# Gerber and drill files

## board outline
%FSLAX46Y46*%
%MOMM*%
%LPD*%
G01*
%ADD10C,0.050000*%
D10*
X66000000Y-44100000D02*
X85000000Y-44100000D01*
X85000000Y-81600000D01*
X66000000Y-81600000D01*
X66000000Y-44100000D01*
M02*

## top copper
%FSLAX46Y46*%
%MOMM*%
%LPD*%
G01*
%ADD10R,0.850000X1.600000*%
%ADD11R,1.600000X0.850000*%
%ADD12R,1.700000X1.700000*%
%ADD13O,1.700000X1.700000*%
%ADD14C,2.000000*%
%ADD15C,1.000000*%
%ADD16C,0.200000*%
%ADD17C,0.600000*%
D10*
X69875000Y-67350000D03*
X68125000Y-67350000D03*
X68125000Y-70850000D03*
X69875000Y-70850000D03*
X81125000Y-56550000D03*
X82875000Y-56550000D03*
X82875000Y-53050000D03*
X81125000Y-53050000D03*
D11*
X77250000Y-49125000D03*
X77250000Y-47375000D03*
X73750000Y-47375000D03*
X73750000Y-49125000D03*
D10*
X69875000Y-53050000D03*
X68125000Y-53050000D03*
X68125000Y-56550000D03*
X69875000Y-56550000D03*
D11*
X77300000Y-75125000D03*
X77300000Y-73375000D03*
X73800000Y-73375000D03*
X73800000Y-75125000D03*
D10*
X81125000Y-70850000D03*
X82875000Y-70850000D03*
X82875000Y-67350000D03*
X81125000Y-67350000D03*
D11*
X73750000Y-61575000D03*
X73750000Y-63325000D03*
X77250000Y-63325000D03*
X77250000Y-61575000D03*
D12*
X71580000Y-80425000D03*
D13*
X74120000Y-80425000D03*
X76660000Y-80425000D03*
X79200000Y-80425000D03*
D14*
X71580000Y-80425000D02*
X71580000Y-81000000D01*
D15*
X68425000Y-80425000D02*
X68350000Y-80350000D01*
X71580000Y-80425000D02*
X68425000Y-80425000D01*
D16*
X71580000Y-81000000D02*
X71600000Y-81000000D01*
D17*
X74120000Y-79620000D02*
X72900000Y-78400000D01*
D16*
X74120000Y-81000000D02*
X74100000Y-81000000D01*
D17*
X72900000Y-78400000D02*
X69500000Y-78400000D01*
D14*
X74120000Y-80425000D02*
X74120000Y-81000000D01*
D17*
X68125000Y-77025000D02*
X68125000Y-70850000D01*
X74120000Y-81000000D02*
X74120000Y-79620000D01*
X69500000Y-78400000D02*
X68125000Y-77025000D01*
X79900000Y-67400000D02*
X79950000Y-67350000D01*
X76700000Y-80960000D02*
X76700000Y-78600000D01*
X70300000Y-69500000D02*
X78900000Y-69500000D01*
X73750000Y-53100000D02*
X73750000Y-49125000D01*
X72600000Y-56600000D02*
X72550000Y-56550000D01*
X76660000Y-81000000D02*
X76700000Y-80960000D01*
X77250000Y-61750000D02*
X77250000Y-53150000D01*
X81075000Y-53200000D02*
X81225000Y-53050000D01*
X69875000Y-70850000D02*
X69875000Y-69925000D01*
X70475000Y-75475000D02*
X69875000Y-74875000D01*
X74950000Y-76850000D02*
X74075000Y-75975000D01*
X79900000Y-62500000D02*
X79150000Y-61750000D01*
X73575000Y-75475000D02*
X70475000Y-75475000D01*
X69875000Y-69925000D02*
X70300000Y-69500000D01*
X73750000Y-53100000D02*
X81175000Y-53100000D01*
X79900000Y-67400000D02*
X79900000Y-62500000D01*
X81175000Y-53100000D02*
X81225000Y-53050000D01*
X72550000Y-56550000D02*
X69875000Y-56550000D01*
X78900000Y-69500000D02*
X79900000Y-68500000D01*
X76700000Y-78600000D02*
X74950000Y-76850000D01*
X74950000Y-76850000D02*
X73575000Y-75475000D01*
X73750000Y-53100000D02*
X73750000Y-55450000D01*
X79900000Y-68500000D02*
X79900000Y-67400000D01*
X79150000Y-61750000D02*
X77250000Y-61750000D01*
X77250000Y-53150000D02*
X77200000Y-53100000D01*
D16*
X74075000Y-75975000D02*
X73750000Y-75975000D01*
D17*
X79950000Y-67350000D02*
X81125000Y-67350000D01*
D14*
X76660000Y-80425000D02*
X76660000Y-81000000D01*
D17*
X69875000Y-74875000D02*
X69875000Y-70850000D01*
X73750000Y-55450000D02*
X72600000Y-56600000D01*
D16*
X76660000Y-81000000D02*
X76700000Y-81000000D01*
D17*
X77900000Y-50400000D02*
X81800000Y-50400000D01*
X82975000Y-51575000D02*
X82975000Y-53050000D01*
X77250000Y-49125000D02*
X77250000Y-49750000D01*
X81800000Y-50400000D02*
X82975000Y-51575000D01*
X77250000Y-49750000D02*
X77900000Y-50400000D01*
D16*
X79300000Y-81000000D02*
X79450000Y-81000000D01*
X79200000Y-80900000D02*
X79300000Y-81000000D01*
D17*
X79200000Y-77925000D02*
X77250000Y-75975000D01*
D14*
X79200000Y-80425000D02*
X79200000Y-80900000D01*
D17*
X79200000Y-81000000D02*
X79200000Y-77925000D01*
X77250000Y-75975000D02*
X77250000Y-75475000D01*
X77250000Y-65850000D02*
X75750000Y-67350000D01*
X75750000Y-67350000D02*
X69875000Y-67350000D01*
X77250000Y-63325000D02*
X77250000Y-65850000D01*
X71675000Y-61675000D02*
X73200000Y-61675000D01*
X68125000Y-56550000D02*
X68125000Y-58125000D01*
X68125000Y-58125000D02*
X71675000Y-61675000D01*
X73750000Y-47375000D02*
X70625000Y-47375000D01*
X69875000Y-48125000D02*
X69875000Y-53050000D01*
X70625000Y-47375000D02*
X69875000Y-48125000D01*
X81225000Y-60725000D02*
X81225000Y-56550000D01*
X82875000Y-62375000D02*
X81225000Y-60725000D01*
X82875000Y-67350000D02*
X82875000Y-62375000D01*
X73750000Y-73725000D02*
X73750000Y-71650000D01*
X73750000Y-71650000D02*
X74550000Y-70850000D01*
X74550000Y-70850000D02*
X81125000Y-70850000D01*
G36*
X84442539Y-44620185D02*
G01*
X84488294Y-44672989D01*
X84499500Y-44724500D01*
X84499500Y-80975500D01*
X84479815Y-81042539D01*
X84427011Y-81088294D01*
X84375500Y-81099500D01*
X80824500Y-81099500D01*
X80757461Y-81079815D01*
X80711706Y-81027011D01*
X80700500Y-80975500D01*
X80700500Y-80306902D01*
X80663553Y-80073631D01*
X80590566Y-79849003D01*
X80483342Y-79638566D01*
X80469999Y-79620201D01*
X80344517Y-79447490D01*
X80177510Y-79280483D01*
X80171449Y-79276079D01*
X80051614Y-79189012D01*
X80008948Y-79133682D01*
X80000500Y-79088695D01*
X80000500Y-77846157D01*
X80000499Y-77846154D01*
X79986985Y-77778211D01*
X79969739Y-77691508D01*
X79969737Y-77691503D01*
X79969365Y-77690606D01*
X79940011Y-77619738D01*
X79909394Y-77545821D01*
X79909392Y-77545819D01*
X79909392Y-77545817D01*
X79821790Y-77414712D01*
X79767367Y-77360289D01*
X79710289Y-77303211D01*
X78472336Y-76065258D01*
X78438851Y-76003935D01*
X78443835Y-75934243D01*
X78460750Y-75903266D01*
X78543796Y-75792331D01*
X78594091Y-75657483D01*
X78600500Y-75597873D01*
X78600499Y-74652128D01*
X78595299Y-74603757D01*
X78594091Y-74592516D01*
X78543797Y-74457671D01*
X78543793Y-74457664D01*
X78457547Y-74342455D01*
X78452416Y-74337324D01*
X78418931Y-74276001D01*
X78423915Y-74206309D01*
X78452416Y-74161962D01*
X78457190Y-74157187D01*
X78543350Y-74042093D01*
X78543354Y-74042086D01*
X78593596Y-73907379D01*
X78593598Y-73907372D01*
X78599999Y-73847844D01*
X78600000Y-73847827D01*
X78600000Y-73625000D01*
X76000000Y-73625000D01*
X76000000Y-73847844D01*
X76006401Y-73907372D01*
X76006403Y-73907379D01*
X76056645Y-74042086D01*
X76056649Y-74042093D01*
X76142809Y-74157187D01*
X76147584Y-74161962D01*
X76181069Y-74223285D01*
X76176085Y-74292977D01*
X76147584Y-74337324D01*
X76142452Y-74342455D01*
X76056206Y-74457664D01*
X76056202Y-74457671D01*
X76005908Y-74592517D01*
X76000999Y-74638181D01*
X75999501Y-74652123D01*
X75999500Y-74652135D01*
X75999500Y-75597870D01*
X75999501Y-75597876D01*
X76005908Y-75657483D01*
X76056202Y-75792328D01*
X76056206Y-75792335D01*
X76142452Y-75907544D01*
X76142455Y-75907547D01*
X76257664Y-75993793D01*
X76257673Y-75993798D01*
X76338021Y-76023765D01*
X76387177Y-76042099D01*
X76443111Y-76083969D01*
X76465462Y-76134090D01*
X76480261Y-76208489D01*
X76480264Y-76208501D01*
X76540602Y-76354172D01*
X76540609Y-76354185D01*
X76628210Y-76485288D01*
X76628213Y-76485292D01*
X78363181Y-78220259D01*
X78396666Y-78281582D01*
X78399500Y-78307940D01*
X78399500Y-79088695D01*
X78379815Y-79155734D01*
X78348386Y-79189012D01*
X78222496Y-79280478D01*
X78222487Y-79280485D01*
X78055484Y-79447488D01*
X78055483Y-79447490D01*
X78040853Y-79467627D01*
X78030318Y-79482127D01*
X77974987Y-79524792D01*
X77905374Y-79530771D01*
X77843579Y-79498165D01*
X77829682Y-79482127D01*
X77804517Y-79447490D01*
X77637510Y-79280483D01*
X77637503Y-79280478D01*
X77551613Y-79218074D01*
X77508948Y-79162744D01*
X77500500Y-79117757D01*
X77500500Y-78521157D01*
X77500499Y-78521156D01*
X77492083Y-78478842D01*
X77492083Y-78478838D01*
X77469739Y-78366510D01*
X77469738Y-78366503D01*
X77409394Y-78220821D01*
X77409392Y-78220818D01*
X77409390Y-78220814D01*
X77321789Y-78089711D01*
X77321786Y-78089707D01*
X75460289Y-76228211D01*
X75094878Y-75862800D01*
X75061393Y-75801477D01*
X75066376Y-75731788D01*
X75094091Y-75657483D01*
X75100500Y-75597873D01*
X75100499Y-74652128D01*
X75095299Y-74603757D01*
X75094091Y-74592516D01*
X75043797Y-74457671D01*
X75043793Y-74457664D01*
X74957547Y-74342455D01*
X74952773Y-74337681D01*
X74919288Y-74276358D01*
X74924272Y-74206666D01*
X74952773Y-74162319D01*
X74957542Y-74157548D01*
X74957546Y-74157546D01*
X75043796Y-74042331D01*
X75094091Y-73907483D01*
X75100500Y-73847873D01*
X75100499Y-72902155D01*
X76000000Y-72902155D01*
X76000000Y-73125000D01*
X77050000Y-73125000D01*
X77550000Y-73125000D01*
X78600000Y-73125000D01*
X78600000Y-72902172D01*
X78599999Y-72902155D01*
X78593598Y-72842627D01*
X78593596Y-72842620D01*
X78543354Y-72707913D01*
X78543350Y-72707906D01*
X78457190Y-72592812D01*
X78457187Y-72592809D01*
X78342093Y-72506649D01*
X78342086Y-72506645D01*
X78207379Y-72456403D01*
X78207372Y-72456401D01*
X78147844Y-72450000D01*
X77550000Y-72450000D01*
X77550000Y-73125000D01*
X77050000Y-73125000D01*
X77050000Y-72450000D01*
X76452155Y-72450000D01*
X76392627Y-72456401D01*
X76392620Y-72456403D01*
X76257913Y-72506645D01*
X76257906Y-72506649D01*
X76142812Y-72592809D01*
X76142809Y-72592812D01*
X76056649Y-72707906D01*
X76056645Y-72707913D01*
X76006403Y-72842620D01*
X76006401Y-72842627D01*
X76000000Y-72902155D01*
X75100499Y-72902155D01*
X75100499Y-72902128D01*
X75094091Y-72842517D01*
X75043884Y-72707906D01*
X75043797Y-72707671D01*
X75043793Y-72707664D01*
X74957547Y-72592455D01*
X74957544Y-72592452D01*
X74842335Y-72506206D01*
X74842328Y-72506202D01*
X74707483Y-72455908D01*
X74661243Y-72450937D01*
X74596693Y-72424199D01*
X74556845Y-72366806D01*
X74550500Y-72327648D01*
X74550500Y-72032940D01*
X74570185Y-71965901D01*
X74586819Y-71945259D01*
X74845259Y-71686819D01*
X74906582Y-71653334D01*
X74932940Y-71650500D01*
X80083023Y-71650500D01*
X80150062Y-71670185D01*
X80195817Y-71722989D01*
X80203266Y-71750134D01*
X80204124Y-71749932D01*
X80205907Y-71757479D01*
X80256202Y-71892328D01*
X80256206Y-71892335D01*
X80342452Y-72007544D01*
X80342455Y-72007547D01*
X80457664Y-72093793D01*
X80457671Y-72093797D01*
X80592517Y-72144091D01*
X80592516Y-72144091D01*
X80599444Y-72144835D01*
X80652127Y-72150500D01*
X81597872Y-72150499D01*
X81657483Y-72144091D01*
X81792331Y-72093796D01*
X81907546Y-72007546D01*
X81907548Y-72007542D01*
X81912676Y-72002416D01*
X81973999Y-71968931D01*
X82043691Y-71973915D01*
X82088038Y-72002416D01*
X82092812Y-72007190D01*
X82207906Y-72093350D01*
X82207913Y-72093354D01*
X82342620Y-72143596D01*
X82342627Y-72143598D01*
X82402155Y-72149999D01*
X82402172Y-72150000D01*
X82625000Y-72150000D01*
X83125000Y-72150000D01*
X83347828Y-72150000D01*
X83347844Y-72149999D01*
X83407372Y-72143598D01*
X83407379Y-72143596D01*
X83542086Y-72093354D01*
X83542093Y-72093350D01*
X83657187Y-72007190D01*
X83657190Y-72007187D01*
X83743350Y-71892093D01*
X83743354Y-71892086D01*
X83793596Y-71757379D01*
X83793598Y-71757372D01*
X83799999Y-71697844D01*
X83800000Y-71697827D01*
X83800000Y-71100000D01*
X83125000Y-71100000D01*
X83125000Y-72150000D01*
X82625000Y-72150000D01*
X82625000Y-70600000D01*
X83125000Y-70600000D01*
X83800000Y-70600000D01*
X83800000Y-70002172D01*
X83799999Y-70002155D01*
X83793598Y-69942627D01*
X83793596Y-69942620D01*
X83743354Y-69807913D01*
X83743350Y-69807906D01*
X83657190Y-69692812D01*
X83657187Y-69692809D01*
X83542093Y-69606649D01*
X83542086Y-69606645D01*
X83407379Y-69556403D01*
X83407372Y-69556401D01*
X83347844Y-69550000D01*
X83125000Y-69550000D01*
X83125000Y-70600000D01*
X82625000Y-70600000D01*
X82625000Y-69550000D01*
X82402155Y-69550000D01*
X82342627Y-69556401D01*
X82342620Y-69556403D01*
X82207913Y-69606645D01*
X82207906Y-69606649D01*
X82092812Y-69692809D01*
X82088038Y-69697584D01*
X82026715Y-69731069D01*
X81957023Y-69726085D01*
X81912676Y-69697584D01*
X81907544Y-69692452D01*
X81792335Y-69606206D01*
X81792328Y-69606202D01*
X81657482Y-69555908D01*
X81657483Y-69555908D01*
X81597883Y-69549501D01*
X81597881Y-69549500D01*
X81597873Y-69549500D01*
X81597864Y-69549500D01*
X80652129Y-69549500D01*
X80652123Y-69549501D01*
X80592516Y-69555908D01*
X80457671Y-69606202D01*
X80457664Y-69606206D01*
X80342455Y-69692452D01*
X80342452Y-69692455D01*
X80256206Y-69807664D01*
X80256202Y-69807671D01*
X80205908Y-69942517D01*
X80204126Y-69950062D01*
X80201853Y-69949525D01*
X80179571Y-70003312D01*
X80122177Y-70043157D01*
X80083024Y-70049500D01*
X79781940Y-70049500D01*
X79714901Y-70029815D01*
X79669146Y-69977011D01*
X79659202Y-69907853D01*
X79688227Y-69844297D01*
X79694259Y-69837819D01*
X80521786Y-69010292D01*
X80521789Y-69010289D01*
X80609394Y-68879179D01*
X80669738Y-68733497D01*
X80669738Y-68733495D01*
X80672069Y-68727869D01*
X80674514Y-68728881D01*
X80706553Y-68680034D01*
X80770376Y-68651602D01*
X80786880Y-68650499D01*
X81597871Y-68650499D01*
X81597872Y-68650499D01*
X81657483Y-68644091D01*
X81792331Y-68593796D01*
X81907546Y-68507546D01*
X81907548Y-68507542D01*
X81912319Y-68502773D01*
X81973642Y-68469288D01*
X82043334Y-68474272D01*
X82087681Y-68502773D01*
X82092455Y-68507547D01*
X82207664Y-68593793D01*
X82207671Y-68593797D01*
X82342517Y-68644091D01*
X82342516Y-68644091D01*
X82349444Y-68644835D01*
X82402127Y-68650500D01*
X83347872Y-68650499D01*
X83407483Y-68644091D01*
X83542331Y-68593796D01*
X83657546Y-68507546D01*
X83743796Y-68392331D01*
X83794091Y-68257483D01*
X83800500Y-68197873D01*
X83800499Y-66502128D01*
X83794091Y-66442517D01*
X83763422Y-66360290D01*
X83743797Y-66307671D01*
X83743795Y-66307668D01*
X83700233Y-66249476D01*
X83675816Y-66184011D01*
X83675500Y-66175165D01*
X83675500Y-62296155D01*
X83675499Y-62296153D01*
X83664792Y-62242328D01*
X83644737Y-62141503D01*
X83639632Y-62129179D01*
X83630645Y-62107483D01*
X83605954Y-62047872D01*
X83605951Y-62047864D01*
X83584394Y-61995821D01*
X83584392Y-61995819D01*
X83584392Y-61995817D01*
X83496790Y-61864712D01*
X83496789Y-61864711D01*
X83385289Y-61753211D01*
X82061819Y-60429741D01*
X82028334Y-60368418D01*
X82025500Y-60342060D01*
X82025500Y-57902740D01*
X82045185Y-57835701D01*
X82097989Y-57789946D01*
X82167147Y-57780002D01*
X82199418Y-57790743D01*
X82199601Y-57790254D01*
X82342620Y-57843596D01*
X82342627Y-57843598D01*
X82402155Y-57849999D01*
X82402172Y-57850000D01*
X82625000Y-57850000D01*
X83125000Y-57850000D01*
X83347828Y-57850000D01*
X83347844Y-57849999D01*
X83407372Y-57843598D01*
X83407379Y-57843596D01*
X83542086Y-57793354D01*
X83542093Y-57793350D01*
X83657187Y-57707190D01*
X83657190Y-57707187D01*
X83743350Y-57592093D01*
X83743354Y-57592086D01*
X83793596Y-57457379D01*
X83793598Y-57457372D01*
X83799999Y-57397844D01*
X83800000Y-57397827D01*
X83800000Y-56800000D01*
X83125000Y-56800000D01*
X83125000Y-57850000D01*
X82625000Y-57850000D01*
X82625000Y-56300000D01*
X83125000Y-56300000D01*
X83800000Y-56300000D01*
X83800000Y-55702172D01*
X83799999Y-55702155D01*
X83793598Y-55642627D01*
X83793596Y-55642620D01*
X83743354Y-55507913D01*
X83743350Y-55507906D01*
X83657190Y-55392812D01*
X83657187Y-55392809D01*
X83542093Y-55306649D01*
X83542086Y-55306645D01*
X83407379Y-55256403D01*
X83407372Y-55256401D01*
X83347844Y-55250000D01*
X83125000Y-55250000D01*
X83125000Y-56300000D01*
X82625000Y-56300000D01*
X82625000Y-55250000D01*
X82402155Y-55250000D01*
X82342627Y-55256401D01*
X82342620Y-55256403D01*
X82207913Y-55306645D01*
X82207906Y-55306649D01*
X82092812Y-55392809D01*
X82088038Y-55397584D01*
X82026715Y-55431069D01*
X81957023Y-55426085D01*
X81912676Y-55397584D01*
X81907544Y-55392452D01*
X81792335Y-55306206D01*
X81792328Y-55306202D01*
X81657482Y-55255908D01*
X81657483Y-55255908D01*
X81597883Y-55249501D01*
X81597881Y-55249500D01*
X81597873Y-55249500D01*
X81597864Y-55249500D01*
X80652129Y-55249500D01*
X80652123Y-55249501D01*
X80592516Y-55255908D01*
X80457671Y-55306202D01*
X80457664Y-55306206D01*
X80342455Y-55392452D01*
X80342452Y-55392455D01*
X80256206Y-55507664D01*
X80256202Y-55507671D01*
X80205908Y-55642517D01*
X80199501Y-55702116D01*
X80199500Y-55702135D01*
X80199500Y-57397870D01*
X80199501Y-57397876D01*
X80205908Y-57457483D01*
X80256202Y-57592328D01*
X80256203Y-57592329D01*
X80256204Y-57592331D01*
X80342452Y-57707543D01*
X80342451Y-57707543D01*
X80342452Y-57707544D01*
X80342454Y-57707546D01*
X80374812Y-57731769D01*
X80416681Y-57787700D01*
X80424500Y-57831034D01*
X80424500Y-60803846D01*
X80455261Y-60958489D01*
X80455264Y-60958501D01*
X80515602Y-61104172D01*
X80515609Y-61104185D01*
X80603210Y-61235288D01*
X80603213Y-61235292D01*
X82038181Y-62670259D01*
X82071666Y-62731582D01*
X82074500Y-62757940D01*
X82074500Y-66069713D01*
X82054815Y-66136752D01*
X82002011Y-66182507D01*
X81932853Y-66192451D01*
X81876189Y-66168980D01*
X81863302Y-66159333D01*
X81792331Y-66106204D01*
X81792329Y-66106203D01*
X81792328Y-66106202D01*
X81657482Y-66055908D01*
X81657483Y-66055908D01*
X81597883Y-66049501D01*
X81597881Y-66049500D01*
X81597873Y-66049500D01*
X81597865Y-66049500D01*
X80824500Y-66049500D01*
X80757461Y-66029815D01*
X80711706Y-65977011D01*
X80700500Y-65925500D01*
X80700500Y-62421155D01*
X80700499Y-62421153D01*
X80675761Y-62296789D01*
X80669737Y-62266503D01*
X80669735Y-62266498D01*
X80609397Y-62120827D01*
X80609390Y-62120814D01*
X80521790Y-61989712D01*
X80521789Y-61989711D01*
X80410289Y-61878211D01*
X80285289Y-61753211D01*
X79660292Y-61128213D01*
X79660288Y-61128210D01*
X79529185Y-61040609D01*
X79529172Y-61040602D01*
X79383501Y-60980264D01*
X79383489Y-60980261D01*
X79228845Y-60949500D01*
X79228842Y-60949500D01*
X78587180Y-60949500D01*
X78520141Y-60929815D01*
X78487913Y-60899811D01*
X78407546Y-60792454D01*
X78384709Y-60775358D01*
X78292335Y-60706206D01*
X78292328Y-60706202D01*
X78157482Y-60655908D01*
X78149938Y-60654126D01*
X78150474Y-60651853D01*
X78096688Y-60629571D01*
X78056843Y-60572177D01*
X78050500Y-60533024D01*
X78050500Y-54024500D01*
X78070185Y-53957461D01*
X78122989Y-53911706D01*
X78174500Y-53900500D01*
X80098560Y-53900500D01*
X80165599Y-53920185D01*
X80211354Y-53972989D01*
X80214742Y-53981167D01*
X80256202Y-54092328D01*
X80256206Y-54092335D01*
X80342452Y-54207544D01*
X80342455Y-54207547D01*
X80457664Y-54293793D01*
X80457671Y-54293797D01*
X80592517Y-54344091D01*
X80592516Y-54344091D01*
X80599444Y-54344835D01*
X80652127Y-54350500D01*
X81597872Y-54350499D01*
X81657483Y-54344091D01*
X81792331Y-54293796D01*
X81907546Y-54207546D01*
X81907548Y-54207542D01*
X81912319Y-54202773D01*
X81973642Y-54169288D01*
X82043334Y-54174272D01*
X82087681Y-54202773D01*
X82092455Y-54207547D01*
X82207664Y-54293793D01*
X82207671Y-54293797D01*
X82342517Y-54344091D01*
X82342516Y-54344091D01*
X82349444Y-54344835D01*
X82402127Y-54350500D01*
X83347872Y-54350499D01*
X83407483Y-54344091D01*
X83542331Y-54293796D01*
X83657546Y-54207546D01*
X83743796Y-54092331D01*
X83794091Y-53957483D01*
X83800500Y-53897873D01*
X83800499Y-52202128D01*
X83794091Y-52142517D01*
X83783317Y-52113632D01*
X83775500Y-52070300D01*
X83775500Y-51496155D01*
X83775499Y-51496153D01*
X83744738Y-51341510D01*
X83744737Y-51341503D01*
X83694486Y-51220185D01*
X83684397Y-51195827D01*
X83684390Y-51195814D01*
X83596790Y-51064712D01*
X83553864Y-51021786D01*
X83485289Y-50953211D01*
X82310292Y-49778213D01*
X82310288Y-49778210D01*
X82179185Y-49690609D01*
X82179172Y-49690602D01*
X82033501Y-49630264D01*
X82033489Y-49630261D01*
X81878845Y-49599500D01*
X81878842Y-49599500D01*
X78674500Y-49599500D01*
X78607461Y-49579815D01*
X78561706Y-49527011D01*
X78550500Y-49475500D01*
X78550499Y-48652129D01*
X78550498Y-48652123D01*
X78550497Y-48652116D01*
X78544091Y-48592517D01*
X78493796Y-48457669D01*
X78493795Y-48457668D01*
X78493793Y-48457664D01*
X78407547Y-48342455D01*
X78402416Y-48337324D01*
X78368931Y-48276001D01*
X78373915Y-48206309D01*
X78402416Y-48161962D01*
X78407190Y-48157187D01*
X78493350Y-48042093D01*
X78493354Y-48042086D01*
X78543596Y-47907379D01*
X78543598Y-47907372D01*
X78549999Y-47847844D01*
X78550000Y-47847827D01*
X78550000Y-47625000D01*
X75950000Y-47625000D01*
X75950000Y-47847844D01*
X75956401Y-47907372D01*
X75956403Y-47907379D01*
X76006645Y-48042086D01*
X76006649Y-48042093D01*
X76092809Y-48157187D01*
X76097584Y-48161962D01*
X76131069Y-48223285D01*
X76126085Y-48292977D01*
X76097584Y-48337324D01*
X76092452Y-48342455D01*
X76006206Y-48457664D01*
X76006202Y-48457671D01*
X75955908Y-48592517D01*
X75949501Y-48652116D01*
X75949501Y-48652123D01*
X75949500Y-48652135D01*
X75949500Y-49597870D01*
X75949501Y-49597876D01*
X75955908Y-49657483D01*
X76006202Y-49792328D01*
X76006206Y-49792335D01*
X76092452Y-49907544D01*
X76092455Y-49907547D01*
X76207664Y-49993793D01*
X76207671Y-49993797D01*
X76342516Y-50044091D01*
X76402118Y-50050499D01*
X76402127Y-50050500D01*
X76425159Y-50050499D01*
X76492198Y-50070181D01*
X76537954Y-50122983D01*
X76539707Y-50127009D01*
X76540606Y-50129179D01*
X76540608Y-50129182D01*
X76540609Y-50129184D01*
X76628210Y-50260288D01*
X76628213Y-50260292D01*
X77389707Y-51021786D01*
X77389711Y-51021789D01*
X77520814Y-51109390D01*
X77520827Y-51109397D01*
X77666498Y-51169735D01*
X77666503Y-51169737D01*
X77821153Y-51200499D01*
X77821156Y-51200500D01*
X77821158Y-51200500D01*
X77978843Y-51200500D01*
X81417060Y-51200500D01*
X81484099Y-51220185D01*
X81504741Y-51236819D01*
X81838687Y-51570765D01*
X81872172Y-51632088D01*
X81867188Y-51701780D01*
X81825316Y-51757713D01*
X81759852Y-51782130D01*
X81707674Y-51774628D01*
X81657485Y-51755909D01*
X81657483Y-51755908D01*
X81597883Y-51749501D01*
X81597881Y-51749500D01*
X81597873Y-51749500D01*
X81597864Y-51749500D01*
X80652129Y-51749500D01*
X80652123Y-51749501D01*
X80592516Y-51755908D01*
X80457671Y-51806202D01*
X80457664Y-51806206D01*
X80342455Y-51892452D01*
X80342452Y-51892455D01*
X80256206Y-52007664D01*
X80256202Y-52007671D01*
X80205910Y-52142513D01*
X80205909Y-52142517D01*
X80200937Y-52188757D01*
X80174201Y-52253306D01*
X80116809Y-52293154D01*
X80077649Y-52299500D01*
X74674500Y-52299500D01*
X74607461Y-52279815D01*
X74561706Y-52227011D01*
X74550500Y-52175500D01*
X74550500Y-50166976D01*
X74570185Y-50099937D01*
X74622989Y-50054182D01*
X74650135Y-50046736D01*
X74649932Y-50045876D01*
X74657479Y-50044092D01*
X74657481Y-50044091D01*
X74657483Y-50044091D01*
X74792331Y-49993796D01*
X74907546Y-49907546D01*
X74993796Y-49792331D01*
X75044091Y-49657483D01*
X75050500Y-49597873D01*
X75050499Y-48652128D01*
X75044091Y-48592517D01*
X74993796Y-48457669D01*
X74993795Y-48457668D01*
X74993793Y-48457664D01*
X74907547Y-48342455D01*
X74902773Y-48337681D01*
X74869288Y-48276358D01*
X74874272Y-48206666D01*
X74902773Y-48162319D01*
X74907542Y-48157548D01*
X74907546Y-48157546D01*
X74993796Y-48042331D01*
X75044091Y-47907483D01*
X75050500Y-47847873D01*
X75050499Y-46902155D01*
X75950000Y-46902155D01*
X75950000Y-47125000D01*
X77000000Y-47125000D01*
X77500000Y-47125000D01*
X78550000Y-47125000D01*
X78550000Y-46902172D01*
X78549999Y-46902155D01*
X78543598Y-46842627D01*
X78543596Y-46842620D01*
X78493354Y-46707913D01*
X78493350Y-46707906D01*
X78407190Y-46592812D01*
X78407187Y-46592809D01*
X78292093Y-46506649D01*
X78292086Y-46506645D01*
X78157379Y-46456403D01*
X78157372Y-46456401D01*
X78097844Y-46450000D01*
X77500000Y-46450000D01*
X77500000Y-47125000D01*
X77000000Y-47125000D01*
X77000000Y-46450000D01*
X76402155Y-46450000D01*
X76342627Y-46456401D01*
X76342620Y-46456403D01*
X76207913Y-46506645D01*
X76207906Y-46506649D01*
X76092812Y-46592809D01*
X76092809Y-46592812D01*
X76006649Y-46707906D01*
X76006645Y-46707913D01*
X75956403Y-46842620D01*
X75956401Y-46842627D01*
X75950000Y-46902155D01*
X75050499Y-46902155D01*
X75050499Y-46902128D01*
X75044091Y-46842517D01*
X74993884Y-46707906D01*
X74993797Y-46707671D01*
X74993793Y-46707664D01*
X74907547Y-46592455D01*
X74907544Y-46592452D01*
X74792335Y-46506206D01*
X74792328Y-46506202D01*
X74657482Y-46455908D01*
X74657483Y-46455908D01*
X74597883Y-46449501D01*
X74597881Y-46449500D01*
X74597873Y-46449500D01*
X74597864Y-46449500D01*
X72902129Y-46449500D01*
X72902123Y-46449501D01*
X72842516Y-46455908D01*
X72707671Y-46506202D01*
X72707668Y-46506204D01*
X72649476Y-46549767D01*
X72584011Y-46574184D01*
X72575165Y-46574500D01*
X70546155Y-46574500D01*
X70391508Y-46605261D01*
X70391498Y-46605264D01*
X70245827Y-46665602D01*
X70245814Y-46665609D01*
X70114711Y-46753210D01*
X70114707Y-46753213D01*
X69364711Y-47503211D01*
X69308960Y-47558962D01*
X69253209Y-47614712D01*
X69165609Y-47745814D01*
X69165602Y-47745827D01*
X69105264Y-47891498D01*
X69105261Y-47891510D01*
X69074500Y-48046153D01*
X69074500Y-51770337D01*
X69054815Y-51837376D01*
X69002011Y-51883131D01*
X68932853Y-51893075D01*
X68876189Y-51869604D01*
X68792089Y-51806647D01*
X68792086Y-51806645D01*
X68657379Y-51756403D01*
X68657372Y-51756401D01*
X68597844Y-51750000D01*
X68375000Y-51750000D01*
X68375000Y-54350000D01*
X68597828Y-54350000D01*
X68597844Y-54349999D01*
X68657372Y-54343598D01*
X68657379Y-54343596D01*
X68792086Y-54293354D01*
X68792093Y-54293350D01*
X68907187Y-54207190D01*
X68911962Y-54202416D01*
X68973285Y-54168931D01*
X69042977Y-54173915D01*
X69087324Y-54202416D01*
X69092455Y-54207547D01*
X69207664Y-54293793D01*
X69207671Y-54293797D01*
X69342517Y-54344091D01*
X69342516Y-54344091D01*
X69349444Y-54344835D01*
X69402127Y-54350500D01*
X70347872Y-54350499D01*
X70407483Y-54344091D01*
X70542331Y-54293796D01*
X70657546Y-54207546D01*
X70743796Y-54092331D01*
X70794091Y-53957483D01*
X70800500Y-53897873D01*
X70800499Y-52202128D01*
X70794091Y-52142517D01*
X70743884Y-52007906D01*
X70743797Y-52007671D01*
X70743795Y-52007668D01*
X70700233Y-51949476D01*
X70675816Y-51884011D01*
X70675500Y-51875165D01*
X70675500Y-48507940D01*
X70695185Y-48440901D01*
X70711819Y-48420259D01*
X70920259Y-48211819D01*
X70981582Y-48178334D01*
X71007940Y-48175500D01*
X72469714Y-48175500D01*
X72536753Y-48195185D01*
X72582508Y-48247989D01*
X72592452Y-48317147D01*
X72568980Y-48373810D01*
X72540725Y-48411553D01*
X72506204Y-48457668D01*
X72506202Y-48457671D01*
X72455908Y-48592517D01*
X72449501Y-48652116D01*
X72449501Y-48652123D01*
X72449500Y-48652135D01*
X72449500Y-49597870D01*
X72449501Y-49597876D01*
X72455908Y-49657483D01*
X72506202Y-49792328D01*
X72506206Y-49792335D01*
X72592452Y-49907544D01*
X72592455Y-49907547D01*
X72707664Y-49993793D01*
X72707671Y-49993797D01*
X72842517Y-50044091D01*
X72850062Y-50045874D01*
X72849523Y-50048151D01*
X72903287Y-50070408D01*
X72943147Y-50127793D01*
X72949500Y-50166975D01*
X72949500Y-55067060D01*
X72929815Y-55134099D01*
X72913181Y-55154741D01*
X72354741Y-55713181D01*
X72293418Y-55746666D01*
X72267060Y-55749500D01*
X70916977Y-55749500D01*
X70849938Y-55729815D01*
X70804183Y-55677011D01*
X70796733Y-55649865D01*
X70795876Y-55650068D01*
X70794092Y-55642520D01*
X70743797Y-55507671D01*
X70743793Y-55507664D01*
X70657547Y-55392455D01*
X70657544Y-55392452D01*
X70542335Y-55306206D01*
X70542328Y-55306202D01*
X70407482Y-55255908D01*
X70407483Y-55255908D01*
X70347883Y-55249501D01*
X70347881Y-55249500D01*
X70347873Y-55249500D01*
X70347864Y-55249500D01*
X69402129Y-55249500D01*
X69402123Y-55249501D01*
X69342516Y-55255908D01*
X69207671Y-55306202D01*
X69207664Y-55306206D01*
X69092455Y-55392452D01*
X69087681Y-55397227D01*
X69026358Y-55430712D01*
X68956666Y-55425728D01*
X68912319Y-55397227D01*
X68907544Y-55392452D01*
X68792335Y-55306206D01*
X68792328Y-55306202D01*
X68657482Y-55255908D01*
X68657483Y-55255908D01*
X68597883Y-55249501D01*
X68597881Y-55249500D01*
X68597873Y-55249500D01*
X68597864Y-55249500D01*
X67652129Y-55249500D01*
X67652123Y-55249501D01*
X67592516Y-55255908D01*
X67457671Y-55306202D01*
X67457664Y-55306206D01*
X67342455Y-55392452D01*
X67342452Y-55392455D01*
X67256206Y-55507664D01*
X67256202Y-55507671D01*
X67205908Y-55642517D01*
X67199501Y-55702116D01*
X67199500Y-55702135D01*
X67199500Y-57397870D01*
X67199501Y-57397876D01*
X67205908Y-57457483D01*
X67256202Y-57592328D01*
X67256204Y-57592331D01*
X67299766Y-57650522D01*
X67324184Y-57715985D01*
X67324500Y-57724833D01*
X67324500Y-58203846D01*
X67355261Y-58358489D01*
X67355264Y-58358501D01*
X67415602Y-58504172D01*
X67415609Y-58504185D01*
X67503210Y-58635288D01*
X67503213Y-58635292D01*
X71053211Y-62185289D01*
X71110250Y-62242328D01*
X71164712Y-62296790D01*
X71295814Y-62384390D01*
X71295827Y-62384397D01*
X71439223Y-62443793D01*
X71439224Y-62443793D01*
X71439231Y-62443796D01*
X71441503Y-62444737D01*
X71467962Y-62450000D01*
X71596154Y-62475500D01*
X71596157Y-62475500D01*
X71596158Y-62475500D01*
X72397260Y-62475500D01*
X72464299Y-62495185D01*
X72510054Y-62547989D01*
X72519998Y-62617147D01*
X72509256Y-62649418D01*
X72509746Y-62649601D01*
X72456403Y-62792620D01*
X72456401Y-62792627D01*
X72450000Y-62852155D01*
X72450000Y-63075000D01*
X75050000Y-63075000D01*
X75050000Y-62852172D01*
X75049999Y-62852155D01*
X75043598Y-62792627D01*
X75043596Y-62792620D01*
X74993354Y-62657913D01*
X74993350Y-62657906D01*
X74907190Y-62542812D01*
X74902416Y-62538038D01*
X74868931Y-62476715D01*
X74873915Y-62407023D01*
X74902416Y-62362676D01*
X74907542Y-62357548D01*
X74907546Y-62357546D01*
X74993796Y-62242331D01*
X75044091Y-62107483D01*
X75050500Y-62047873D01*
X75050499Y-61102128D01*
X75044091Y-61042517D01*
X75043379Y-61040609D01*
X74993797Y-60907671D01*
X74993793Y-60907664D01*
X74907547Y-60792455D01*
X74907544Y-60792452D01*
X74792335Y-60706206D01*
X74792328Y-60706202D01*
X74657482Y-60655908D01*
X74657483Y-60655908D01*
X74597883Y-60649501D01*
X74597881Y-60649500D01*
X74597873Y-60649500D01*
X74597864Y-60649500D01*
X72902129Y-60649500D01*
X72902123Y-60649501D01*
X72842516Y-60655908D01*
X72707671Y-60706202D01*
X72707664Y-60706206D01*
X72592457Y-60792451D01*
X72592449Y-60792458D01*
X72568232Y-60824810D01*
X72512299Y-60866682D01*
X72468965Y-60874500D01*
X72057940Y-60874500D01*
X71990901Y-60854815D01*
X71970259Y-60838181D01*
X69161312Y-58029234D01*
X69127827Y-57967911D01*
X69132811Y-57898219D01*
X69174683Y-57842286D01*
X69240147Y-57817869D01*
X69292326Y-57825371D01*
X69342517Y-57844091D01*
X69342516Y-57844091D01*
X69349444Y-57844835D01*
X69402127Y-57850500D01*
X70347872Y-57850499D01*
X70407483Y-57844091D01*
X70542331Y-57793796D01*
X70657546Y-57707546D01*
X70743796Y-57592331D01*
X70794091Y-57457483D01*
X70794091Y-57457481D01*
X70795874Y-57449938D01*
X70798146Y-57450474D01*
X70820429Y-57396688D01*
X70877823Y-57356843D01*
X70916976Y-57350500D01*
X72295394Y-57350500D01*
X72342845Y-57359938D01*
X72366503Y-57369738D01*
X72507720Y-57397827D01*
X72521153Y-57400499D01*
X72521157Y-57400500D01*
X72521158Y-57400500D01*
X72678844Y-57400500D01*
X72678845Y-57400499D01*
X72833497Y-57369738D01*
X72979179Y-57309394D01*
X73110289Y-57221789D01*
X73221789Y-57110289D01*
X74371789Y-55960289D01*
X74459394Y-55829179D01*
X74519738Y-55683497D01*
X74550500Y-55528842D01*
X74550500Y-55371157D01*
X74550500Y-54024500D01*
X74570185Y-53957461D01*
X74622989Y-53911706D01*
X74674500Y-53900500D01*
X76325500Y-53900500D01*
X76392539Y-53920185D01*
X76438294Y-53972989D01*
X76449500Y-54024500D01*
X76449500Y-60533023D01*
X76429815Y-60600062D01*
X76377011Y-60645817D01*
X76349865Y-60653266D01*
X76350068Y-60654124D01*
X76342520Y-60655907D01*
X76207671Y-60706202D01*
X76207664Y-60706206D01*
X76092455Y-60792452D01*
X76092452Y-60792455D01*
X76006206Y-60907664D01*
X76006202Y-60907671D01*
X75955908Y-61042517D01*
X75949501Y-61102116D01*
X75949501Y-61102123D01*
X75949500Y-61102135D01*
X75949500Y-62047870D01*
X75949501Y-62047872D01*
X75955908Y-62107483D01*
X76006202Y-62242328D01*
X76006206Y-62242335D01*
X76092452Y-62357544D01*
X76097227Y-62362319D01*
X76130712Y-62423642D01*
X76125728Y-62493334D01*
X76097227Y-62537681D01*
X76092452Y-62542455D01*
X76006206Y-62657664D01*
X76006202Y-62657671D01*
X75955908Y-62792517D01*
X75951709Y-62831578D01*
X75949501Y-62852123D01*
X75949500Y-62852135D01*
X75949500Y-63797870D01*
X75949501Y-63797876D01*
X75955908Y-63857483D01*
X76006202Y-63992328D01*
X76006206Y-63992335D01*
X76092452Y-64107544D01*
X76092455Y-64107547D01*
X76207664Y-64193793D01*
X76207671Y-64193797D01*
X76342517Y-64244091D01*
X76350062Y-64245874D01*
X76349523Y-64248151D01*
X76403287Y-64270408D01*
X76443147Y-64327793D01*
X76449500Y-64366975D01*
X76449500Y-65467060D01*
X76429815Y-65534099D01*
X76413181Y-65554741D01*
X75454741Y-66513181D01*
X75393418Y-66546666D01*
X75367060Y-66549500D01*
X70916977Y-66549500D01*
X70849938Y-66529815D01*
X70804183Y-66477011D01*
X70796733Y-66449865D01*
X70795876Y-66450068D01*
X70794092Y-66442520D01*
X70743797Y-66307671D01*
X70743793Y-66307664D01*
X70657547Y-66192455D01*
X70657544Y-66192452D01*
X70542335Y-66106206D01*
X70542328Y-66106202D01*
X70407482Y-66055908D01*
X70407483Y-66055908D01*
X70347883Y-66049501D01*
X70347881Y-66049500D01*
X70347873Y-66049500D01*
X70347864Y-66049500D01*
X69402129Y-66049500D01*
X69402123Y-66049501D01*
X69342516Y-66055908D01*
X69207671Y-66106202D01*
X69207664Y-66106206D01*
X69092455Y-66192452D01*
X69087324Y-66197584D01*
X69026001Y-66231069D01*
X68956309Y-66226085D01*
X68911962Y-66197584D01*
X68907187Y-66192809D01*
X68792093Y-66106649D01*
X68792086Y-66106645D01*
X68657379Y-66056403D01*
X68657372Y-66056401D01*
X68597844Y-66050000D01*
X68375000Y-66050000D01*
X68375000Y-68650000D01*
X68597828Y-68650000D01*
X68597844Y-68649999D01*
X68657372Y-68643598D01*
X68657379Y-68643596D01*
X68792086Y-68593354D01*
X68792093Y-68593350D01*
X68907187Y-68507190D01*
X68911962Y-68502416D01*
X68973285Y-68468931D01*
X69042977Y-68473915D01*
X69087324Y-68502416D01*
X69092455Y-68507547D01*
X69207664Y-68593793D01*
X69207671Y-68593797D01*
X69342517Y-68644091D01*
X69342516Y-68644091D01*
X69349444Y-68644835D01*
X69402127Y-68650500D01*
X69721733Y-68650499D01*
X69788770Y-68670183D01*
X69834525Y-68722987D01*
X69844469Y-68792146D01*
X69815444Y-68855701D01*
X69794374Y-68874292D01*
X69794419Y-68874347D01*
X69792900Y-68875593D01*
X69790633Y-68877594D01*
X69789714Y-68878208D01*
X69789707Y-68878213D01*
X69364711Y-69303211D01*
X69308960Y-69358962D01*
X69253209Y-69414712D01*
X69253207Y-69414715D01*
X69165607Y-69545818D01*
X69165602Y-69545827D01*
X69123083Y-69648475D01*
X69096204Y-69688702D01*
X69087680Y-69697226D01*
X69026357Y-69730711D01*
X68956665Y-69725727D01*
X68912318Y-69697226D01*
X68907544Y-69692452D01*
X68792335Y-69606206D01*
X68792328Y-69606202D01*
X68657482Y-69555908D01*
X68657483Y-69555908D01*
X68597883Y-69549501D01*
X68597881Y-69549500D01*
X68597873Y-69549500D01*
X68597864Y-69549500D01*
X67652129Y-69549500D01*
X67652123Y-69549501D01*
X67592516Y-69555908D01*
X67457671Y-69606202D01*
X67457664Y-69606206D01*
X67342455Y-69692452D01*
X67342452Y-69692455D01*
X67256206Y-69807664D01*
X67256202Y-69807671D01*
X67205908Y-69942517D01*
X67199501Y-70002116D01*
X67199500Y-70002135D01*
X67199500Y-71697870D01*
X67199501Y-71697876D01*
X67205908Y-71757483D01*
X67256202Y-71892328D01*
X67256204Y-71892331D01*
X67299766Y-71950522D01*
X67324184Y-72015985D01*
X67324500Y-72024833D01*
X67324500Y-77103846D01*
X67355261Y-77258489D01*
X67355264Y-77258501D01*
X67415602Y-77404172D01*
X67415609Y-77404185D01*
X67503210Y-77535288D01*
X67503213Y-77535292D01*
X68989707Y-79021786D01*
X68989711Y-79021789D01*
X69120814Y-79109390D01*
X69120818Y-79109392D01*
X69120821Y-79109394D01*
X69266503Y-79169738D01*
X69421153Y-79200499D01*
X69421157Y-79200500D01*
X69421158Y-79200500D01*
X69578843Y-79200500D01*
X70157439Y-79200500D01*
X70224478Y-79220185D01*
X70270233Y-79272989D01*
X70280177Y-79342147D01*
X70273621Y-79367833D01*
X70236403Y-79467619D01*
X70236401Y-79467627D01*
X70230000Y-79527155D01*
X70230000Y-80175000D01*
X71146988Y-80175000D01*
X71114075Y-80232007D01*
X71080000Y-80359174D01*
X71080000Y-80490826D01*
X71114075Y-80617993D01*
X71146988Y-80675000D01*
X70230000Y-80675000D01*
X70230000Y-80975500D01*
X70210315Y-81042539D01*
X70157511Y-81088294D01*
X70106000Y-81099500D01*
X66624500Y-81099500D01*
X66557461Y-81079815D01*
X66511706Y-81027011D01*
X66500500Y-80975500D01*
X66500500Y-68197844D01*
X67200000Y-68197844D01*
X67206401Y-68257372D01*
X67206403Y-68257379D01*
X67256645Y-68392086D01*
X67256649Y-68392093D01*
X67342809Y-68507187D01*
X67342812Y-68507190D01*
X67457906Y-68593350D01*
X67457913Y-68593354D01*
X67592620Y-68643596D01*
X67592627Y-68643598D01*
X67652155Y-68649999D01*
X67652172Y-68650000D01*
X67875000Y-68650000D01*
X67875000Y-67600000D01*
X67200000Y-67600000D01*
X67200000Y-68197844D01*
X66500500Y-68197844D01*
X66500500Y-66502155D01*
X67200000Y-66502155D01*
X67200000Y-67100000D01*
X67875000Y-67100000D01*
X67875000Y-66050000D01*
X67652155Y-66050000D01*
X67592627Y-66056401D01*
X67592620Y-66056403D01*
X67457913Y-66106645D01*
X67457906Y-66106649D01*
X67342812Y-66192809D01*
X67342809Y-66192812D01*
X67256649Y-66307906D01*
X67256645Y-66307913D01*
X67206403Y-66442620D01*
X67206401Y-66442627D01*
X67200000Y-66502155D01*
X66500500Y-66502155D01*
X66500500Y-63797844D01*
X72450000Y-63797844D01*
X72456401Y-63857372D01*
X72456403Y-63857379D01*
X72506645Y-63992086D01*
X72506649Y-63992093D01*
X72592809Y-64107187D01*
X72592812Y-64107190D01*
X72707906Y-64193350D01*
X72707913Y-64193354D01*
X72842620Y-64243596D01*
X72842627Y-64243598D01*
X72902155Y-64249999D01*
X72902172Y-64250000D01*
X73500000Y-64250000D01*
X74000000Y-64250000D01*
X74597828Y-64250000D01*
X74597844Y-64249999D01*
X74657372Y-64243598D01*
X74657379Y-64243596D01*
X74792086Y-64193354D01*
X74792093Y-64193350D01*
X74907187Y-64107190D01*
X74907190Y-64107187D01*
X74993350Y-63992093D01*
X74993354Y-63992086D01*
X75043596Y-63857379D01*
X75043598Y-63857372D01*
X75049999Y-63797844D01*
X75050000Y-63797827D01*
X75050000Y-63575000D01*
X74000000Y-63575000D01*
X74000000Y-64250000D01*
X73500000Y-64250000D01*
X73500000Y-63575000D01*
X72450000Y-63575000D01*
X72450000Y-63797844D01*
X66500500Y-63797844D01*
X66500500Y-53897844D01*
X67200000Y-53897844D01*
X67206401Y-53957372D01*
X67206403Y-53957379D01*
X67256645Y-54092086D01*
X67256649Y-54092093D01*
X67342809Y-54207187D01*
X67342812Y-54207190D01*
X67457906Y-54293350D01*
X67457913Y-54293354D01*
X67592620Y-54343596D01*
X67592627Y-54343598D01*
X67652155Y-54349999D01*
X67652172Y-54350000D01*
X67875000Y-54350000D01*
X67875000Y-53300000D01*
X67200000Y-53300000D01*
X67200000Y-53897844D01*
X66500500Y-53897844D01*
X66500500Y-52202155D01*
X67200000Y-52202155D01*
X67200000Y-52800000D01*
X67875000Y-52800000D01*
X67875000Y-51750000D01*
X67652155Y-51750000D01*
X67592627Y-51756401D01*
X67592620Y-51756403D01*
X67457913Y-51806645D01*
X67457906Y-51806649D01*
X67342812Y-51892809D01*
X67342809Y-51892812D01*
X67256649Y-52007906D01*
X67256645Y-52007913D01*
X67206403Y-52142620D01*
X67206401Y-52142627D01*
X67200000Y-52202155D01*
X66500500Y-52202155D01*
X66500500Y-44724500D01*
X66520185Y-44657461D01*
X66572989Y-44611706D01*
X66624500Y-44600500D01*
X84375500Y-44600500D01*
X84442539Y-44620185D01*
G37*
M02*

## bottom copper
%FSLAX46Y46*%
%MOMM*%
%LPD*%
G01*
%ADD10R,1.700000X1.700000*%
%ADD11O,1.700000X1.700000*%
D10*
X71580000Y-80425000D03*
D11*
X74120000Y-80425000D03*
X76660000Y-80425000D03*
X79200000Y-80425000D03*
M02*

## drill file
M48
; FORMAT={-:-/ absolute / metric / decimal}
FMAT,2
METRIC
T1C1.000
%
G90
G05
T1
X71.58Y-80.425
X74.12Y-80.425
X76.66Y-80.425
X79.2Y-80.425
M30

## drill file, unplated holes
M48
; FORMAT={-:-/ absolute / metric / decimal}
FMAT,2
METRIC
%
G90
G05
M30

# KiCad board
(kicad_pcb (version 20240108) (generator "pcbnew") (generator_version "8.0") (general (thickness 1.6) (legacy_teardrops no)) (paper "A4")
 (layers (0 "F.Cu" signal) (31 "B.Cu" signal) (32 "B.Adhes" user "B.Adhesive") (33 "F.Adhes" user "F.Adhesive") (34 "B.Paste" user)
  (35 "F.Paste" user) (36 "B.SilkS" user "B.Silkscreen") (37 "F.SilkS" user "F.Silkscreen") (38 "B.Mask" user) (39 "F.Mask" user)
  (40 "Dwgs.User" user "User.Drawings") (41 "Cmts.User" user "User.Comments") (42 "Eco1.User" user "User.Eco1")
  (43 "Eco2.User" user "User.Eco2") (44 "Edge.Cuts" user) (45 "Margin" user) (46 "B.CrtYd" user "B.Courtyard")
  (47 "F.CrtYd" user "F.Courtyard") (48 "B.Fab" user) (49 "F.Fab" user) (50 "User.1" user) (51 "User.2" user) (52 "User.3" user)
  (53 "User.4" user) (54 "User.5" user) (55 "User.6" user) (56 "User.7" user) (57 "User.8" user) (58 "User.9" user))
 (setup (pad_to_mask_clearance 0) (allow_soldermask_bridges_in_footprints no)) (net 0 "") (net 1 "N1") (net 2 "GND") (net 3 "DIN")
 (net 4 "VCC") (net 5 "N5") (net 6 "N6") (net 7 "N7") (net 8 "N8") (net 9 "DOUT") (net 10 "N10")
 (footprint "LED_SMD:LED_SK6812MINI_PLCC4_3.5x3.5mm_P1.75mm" (layer "F.Cu") (at 69 69.1 -90)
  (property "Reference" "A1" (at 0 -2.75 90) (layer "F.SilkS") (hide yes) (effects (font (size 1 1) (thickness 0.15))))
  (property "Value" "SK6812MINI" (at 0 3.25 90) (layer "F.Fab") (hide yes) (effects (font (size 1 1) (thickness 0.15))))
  (pad "1" smd rect (at -1.75 -0.875 270) (size 1.6 0.85) (layers "F.Cu" "F.Paste" "F.Mask") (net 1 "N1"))
  (pad "2" smd rect (at -1.75 0.875 270) (size 1.6 0.85) (layers "F.Cu" "F.Paste" "F.Mask") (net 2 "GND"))
  (pad "3" smd rect (at 1.75 0.875 270) (size 1.6 0.85) (layers "F.Cu" "F.Paste" "F.Mask") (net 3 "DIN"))
  (pad "4" smd rect (at 1.75 -0.875 270) (size 1.6 0.85) (layers "F.Cu" "F.Paste" "F.Mask") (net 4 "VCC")))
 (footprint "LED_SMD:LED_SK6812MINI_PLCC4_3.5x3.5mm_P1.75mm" (layer "F.Cu") (at 82 54.8 90)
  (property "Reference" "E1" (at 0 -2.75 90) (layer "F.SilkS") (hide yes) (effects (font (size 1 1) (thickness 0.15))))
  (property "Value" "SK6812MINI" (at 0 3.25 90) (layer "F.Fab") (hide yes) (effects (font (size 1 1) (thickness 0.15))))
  (pad "1" smd rect (at -1.75 -0.875 90) (size 1.6 0.85) (layers "F.Cu" "F.Paste" "F.Mask") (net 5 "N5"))
  (pad "2" smd rect (at -1.75 0.875 90) (size 1.6 0.85) (layers "F.Cu" "F.Paste" "F.Mask") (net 2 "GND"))
  (pad "3" smd rect (at 1.75 0.875 90) (size 1.6 0.85) (layers "F.Cu" "F.Paste" "F.Mask") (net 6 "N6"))
  (pad "4" smd rect (at 1.75 -0.875 90) (size 1.6 0.85) (layers "F.Cu" "F.Paste" "F.Mask") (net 4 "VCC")))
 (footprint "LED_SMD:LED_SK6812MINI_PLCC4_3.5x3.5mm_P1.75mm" (layer "F.Cu") (at 75.5 48.25 180)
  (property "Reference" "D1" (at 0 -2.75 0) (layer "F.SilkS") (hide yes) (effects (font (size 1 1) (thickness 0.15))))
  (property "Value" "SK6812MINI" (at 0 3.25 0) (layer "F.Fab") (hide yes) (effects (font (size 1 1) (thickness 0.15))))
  (pad "1" smd rect (at -1.75 -0.875 180) (size 1.6 0.85) (layers "F.Cu" "F.Paste" "F.Mask") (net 6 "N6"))
  (pad "2" smd rect (at -1.75 0.875 180) (size 1.6 0.85) (layers "F.Cu" "F.Paste" "F.Mask") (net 2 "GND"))
  (pad "3" smd rect (at 1.75 0.875 180) (size 1.6 0.85) (layers "F.Cu" "F.Paste" "F.Mask") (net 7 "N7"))
  (pad "4" smd rect (at 1.75 -0.875 180) (size 1.6 0.85) (layers "F.Cu" "F.Paste" "F.Mask") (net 4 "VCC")))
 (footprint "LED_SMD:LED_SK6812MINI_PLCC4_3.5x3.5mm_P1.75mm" (layer "F.Cu") (at 69 54.8 -90)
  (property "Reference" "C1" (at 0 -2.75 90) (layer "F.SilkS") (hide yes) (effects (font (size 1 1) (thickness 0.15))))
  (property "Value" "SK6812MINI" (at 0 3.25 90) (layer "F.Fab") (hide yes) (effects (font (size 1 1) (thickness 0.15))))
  (pad "1" smd rect (at -1.75 -0.875 270) (size 1.6 0.85) (layers "F.Cu" "F.Paste" "F.Mask") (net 7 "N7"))
  (pad "2" smd rect (at -1.75 0.875 270) (size 1.6 0.85) (layers "F.Cu" "F.Paste" "F.Mask") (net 2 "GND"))
  (pad "3" smd rect (at 1.75 0.875 270) (size 1.6 0.85) (layers "F.Cu" "F.Paste" "F.Mask") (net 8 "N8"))
  (pad "4" smd rect (at 1.75 -0.875 270) (size 1.6 0.85) (layers "F.Cu" "F.Paste" "F.Mask") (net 4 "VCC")))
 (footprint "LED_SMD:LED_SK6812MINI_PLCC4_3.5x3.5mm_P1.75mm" (layer "F.Cu") (at 75.55 74.25 180)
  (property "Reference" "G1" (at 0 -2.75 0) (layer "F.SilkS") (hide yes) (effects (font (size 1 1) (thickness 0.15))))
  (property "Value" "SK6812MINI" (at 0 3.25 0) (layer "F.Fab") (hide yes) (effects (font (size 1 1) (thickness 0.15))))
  (pad "1" smd rect (at -1.75 -0.875 180) (size 1.6 0.85) (layers "F.Cu" "F.Paste" "F.Mask") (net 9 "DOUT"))
  (pad "2" smd rect (at -1.75 0.875 180) (size 1.6 0.85) (layers "F.Cu" "F.Paste" "F.Mask") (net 2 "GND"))
  (pad "3" smd rect (at 1.75 0.875 180) (size 1.6 0.85) (layers "F.Cu" "F.Paste" "F.Mask") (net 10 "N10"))
  (pad "4" smd rect (at 1.75 -0.875 180) (size 1.6 0.85) (layers "F.Cu" "F.Paste" "F.Mask") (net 4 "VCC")))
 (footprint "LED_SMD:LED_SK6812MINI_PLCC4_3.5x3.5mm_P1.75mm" (layer "F.Cu") (at 82 69.1 90)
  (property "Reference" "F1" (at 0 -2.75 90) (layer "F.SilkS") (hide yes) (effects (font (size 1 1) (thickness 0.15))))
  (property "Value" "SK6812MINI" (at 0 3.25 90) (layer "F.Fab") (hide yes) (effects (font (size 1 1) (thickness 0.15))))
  (pad "1" smd rect (at -1.75 -0.875 90) (size 1.6 0.85) (layers "F.Cu" "F.Paste" "F.Mask") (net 10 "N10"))
  (pad "2" smd rect (at -1.75 0.875 90) (size 1.6 0.85) (layers "F.Cu" "F.Paste" "F.Mask") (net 2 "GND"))
  (pad "3" smd rect (at 1.75 0.875 90) (size 1.6 0.85) (layers "F.Cu" "F.Paste" "F.Mask") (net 5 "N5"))
  (pad "4" smd rect (at 1.75 -0.875 90) (size 1.6 0.85) (layers "F.Cu" "F.Paste" "F.Mask") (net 4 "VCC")))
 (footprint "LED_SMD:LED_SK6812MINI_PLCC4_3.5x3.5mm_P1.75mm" (layer "F.Cu") (at 75.5 62.45)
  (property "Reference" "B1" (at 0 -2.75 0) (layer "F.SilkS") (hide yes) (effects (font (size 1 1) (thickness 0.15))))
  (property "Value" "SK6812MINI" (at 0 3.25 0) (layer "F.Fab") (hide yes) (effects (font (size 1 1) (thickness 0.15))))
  (pad "1" smd rect (at -1.75 -0.875) (size 1.6 0.85) (layers "F.Cu" "F.Paste" "F.Mask") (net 8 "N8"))
  (pad "2" smd rect (at -1.75 0.875) (size 1.6 0.85) (layers "F.Cu" "F.Paste" "F.Mask") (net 2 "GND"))
  (pad "3" smd rect (at 1.75 0.875) (size 1.6 0.85) (layers "F.Cu" "F.Paste" "F.Mask") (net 1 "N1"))
  (pad "4" smd rect (at 1.75 -0.875) (size 1.6 0.85) (layers "F.Cu" "F.Paste" "F.Mask") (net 4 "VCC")))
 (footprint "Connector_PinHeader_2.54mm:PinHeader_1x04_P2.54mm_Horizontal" (layer "B.Cu") (at 71.58 80.425 -90)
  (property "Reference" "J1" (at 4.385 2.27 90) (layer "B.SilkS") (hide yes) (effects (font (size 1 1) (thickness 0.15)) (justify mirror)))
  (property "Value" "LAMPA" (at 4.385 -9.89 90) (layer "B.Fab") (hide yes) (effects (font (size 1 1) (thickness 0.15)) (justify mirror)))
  (pad "1" thru_hole rect (at 0 0 270) (size 1.7 1.7) (drill 1) (layers "*.Cu" "*.Mask") (remove_unused_layers no) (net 2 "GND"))
  (pad "2" thru_hole oval (at 0 -2.54 270) (size 1.7 1.7) (drill 1) (layers "*.Cu" "*.Mask") (remove_unused_layers no) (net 3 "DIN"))
  (pad "3" thru_hole oval (at 0 -5.08 270) (size 1.7 1.7) (drill 1) (layers "*.Cu" "*.Mask") (remove_unused_layers no) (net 4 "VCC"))
  (pad "4" thru_hole oval (at 0 -7.62 270) (size 1.7 1.7) (drill 1) (layers "*.Cu" "*.Mask") (remove_unused_layers no) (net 9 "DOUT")))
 (gr_rect (start 66 44.1) (end 85 81.6) (stroke (width 0.05) (type default)) (fill none) (layer "Edge.Cuts"))
 (segment (start 71.58 80.425) (end 71.58 81) (width 2) (layer "F.Cu") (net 2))
 (segment (start 68.425 80.425) (end 68.35 80.35) (width 1) (layer "F.Cu") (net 2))
 (segment (start 71.58 80.425) (end 68.425 80.425) (width 1) (layer "F.Cu") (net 2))
 (segment (start 71.58 81) (end 71.6 81) (width 0.2) (layer "F.Cu") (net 2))
 (segment (start 74.12 79.62) (end 72.9 78.4) (width 0.6) (layer "F.Cu") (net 3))
 (segment (start 74.12 81) (end 74.1 81) (width 0.2) (layer "F.Cu") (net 3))
 (segment (start 72.9 78.4) (end 69.5 78.4) (width 0.6) (layer "F.Cu") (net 3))
 (segment (start 74.12 80.425) (end 74.12 81) (width 2) (layer "F.Cu") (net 3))
 (segment (start 68.125 77.025) (end 68.125 70.85) (width 0.6) (layer "F.Cu") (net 3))
 (segment (start 74.12 81) (end 74.12 79.62) (width 0.6) (layer "F.Cu") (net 3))
 (segment (start 69.5 78.4) (end 68.125 77.025) (width 0.6) (layer "F.Cu") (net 3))
 (segment (start 79.9 67.4) (end 79.95 67.35) (width 0.6) (layer "F.Cu") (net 4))
 (segment (start 76.7 80.96) (end 76.7 78.6) (width 0.6) (layer "F.Cu") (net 4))
 (segment (start 70.3 69.5) (end 78.9 69.5) (width 0.6) (layer "F.Cu") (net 4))
 (segment (start 73.75 53.1) (end 73.75 49.125) (width 0.6) (layer "F.Cu") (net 4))
 (segment (start 72.6 56.6) (end 72.55 56.55) (width 0.6) (layer "F.Cu") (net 4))
 (segment (start 76.66 81) (end 76.7 80.96) (width 0.6) (layer "F.Cu") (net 4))
 (segment (start 77.25 61.75) (end 77.25 53.15) (width 0.6) (layer "F.Cu") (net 4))
 (segment (start 81.075 53.2) (end 81.225 53.05) (width 0.6) (layer "F.Cu") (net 4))
 (segment (start 69.875 70.85) (end 69.875 69.925) (width 0.6) (layer "F.Cu") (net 4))
 (segment (start 70.475 75.475) (end 69.875 74.875) (width 0.6) (layer "F.Cu") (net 4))
 (segment (start 74.95 76.85) (end 74.075 75.975) (width 0.6) (layer "F.Cu") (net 4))
 (segment (start 79.9 62.5) (end 79.15 61.75) (width 0.6) (layer "F.Cu") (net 4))
 (segment (start 73.575 75.475) (end 70.475 75.475) (width 0.6) (layer "F.Cu") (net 4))
 (segment (start 69.875 69.925) (end 70.3 69.5) (width 0.6) (layer "F.Cu") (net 4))
 (segment (start 73.75 53.1) (end 81.175 53.1) (width 0.6) (layer "F.Cu") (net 4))
 (segment (start 79.9 67.4) (end 79.9 62.5) (width 0.6) (layer "F.Cu") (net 4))
 (segment (start 81.175 53.1) (end 81.225 53.05) (width 0.6) (layer "F.Cu") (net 4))
 (segment (start 72.55 56.55) (end 69.875 56.55) (width 0.6) (layer "F.Cu") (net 4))
 (segment (start 78.9 69.5) (end 79.9 68.5) (width 0.6) (layer "F.Cu") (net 4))
 (segment (start 76.7 78.6) (end 74.95 76.85) (width 0.6) (layer "F.Cu") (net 4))
 (segment (start 74.95 76.85) (end 73.575 75.475) (width 0.6) (layer "F.Cu") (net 4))
 (segment (start 73.75 53.1) (end 73.75 55.45) (width 0.6) (layer "F.Cu") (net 4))
 (segment (start 79.9 68.5) (end 79.9 67.4) (width 0.6) (layer "F.Cu") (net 4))
 (segment (start 79.15 61.75) (end 77.25 61.75) (width 0.6) (layer "F.Cu") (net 4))
 (segment (start 77.25 53.15) (end 77.2 53.1) (width 0.6) (layer "F.Cu") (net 4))
 (segment (start 74.075 75.975) (end 73.75 75.975) (width 0.2) (layer "F.Cu") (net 4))
 (segment (start 79.95 67.35) (end 81.125 67.35) (width 0.6) (layer "F.Cu") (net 4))
 (segment (start 76.66 80.425) (end 76.66 81) (width 2) (layer "F.Cu") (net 4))
 (segment (start 69.875 74.875) (end 69.875 70.85) (width 0.6) (layer "F.Cu") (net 4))
 (segment (start 73.75 55.45) (end 72.6 56.6) (width 0.6) (layer "F.Cu") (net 4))
 (segment (start 76.66 81) (end 76.7 81) (width 0.2) (layer "F.Cu") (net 4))
 (segment (start 77.9 50.4) (end 81.8 50.4) (width 0.6) (layer "F.Cu") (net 6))
 (segment (start 82.975 51.575) (end 82.975 53.05) (width 0.6) (layer "F.Cu") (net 6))
 (segment (start 77.25 49.125) (end 77.25 49.75) (width 0.6) (layer "F.Cu") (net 6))
 (segment (start 81.8 50.4) (end 82.975 51.575) (width 0.6) (layer "F.Cu") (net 6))
 (segment (start 77.25 49.75) (end 77.9 50.4) (width 0.6) (layer "F.Cu") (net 6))
 (segment (start 79.3 81) (end 79.45 81) (width 0.2) (layer "F.Cu") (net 9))
 (segment (start 79.2 80.9) (end 79.3 81) (width 0.2) (layer "F.Cu") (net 9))
 (segment (start 79.2 77.925) (end 77.25 75.975) (width 0.6) (layer "F.Cu") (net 9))
 (segment (start 79.2 80.425) (end 79.2 80.9) (width 2) (layer "F.Cu") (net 9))
 (segment (start 79.2 81) (end 79.2 77.925) (width 0.6) (layer "F.Cu") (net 9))
 (segment (start 77.25 75.975) (end 77.25 75.475) (width 0.6) (layer "F.Cu") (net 9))
 (segment (start 77.25 65.85) (end 75.75 67.35) (width 0.6) (layer "F.Cu") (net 1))
 (segment (start 75.75 67.35) (end 69.875 67.35) (width 0.6) (layer "F.Cu") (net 1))
 (segment (start 77.25 63.325) (end 77.25 65.85) (width 0.6) (layer "F.Cu") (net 1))
 (segment (start 71.675 61.675) (end 73.2 61.675) (width 0.6) (layer "F.Cu") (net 8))
 (segment (start 68.125 56.55) (end 68.125 58.125) (width 0.6) (layer "F.Cu") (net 8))
 (segment (start 68.125 58.125) (end 71.675 61.675) (width 0.6) (layer "F.Cu") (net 8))
 (segment (start 73.75 47.375) (end 70.625 47.375) (width 0.6) (layer "F.Cu") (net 7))
 (segment (start 69.875 48.125) (end 69.875 53.05) (width 0.6) (layer "F.Cu") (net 7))
 (segment (start 70.625 47.375) (end 69.875 48.125) (width 0.6) (layer "F.Cu") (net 7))
 (segment (start 81.225 60.725) (end 81.225 56.55) (width 0.6) (layer "F.Cu") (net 5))
 (segment (start 82.875 62.375) (end 81.225 60.725) (width 0.6) (layer "F.Cu") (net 5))
 (segment (start 82.875 67.35) (end 82.875 62.375) (width 0.6) (layer "F.Cu") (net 5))
 (segment (start 73.75 73.725) (end 73.75 71.65) (width 0.6) (layer "F.Cu") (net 10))
 (segment (start 73.75 71.65) (end 74.55 70.85) (width 0.6) (layer "F.Cu") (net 10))
 (segment (start 74.55 70.85) (end 81.125 70.85) (width 0.6) (layer "F.Cu") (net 10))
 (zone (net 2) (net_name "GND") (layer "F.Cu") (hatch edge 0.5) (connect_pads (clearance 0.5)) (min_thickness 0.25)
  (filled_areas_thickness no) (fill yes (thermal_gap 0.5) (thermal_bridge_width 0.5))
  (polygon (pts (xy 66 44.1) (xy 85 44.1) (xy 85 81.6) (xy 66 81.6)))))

